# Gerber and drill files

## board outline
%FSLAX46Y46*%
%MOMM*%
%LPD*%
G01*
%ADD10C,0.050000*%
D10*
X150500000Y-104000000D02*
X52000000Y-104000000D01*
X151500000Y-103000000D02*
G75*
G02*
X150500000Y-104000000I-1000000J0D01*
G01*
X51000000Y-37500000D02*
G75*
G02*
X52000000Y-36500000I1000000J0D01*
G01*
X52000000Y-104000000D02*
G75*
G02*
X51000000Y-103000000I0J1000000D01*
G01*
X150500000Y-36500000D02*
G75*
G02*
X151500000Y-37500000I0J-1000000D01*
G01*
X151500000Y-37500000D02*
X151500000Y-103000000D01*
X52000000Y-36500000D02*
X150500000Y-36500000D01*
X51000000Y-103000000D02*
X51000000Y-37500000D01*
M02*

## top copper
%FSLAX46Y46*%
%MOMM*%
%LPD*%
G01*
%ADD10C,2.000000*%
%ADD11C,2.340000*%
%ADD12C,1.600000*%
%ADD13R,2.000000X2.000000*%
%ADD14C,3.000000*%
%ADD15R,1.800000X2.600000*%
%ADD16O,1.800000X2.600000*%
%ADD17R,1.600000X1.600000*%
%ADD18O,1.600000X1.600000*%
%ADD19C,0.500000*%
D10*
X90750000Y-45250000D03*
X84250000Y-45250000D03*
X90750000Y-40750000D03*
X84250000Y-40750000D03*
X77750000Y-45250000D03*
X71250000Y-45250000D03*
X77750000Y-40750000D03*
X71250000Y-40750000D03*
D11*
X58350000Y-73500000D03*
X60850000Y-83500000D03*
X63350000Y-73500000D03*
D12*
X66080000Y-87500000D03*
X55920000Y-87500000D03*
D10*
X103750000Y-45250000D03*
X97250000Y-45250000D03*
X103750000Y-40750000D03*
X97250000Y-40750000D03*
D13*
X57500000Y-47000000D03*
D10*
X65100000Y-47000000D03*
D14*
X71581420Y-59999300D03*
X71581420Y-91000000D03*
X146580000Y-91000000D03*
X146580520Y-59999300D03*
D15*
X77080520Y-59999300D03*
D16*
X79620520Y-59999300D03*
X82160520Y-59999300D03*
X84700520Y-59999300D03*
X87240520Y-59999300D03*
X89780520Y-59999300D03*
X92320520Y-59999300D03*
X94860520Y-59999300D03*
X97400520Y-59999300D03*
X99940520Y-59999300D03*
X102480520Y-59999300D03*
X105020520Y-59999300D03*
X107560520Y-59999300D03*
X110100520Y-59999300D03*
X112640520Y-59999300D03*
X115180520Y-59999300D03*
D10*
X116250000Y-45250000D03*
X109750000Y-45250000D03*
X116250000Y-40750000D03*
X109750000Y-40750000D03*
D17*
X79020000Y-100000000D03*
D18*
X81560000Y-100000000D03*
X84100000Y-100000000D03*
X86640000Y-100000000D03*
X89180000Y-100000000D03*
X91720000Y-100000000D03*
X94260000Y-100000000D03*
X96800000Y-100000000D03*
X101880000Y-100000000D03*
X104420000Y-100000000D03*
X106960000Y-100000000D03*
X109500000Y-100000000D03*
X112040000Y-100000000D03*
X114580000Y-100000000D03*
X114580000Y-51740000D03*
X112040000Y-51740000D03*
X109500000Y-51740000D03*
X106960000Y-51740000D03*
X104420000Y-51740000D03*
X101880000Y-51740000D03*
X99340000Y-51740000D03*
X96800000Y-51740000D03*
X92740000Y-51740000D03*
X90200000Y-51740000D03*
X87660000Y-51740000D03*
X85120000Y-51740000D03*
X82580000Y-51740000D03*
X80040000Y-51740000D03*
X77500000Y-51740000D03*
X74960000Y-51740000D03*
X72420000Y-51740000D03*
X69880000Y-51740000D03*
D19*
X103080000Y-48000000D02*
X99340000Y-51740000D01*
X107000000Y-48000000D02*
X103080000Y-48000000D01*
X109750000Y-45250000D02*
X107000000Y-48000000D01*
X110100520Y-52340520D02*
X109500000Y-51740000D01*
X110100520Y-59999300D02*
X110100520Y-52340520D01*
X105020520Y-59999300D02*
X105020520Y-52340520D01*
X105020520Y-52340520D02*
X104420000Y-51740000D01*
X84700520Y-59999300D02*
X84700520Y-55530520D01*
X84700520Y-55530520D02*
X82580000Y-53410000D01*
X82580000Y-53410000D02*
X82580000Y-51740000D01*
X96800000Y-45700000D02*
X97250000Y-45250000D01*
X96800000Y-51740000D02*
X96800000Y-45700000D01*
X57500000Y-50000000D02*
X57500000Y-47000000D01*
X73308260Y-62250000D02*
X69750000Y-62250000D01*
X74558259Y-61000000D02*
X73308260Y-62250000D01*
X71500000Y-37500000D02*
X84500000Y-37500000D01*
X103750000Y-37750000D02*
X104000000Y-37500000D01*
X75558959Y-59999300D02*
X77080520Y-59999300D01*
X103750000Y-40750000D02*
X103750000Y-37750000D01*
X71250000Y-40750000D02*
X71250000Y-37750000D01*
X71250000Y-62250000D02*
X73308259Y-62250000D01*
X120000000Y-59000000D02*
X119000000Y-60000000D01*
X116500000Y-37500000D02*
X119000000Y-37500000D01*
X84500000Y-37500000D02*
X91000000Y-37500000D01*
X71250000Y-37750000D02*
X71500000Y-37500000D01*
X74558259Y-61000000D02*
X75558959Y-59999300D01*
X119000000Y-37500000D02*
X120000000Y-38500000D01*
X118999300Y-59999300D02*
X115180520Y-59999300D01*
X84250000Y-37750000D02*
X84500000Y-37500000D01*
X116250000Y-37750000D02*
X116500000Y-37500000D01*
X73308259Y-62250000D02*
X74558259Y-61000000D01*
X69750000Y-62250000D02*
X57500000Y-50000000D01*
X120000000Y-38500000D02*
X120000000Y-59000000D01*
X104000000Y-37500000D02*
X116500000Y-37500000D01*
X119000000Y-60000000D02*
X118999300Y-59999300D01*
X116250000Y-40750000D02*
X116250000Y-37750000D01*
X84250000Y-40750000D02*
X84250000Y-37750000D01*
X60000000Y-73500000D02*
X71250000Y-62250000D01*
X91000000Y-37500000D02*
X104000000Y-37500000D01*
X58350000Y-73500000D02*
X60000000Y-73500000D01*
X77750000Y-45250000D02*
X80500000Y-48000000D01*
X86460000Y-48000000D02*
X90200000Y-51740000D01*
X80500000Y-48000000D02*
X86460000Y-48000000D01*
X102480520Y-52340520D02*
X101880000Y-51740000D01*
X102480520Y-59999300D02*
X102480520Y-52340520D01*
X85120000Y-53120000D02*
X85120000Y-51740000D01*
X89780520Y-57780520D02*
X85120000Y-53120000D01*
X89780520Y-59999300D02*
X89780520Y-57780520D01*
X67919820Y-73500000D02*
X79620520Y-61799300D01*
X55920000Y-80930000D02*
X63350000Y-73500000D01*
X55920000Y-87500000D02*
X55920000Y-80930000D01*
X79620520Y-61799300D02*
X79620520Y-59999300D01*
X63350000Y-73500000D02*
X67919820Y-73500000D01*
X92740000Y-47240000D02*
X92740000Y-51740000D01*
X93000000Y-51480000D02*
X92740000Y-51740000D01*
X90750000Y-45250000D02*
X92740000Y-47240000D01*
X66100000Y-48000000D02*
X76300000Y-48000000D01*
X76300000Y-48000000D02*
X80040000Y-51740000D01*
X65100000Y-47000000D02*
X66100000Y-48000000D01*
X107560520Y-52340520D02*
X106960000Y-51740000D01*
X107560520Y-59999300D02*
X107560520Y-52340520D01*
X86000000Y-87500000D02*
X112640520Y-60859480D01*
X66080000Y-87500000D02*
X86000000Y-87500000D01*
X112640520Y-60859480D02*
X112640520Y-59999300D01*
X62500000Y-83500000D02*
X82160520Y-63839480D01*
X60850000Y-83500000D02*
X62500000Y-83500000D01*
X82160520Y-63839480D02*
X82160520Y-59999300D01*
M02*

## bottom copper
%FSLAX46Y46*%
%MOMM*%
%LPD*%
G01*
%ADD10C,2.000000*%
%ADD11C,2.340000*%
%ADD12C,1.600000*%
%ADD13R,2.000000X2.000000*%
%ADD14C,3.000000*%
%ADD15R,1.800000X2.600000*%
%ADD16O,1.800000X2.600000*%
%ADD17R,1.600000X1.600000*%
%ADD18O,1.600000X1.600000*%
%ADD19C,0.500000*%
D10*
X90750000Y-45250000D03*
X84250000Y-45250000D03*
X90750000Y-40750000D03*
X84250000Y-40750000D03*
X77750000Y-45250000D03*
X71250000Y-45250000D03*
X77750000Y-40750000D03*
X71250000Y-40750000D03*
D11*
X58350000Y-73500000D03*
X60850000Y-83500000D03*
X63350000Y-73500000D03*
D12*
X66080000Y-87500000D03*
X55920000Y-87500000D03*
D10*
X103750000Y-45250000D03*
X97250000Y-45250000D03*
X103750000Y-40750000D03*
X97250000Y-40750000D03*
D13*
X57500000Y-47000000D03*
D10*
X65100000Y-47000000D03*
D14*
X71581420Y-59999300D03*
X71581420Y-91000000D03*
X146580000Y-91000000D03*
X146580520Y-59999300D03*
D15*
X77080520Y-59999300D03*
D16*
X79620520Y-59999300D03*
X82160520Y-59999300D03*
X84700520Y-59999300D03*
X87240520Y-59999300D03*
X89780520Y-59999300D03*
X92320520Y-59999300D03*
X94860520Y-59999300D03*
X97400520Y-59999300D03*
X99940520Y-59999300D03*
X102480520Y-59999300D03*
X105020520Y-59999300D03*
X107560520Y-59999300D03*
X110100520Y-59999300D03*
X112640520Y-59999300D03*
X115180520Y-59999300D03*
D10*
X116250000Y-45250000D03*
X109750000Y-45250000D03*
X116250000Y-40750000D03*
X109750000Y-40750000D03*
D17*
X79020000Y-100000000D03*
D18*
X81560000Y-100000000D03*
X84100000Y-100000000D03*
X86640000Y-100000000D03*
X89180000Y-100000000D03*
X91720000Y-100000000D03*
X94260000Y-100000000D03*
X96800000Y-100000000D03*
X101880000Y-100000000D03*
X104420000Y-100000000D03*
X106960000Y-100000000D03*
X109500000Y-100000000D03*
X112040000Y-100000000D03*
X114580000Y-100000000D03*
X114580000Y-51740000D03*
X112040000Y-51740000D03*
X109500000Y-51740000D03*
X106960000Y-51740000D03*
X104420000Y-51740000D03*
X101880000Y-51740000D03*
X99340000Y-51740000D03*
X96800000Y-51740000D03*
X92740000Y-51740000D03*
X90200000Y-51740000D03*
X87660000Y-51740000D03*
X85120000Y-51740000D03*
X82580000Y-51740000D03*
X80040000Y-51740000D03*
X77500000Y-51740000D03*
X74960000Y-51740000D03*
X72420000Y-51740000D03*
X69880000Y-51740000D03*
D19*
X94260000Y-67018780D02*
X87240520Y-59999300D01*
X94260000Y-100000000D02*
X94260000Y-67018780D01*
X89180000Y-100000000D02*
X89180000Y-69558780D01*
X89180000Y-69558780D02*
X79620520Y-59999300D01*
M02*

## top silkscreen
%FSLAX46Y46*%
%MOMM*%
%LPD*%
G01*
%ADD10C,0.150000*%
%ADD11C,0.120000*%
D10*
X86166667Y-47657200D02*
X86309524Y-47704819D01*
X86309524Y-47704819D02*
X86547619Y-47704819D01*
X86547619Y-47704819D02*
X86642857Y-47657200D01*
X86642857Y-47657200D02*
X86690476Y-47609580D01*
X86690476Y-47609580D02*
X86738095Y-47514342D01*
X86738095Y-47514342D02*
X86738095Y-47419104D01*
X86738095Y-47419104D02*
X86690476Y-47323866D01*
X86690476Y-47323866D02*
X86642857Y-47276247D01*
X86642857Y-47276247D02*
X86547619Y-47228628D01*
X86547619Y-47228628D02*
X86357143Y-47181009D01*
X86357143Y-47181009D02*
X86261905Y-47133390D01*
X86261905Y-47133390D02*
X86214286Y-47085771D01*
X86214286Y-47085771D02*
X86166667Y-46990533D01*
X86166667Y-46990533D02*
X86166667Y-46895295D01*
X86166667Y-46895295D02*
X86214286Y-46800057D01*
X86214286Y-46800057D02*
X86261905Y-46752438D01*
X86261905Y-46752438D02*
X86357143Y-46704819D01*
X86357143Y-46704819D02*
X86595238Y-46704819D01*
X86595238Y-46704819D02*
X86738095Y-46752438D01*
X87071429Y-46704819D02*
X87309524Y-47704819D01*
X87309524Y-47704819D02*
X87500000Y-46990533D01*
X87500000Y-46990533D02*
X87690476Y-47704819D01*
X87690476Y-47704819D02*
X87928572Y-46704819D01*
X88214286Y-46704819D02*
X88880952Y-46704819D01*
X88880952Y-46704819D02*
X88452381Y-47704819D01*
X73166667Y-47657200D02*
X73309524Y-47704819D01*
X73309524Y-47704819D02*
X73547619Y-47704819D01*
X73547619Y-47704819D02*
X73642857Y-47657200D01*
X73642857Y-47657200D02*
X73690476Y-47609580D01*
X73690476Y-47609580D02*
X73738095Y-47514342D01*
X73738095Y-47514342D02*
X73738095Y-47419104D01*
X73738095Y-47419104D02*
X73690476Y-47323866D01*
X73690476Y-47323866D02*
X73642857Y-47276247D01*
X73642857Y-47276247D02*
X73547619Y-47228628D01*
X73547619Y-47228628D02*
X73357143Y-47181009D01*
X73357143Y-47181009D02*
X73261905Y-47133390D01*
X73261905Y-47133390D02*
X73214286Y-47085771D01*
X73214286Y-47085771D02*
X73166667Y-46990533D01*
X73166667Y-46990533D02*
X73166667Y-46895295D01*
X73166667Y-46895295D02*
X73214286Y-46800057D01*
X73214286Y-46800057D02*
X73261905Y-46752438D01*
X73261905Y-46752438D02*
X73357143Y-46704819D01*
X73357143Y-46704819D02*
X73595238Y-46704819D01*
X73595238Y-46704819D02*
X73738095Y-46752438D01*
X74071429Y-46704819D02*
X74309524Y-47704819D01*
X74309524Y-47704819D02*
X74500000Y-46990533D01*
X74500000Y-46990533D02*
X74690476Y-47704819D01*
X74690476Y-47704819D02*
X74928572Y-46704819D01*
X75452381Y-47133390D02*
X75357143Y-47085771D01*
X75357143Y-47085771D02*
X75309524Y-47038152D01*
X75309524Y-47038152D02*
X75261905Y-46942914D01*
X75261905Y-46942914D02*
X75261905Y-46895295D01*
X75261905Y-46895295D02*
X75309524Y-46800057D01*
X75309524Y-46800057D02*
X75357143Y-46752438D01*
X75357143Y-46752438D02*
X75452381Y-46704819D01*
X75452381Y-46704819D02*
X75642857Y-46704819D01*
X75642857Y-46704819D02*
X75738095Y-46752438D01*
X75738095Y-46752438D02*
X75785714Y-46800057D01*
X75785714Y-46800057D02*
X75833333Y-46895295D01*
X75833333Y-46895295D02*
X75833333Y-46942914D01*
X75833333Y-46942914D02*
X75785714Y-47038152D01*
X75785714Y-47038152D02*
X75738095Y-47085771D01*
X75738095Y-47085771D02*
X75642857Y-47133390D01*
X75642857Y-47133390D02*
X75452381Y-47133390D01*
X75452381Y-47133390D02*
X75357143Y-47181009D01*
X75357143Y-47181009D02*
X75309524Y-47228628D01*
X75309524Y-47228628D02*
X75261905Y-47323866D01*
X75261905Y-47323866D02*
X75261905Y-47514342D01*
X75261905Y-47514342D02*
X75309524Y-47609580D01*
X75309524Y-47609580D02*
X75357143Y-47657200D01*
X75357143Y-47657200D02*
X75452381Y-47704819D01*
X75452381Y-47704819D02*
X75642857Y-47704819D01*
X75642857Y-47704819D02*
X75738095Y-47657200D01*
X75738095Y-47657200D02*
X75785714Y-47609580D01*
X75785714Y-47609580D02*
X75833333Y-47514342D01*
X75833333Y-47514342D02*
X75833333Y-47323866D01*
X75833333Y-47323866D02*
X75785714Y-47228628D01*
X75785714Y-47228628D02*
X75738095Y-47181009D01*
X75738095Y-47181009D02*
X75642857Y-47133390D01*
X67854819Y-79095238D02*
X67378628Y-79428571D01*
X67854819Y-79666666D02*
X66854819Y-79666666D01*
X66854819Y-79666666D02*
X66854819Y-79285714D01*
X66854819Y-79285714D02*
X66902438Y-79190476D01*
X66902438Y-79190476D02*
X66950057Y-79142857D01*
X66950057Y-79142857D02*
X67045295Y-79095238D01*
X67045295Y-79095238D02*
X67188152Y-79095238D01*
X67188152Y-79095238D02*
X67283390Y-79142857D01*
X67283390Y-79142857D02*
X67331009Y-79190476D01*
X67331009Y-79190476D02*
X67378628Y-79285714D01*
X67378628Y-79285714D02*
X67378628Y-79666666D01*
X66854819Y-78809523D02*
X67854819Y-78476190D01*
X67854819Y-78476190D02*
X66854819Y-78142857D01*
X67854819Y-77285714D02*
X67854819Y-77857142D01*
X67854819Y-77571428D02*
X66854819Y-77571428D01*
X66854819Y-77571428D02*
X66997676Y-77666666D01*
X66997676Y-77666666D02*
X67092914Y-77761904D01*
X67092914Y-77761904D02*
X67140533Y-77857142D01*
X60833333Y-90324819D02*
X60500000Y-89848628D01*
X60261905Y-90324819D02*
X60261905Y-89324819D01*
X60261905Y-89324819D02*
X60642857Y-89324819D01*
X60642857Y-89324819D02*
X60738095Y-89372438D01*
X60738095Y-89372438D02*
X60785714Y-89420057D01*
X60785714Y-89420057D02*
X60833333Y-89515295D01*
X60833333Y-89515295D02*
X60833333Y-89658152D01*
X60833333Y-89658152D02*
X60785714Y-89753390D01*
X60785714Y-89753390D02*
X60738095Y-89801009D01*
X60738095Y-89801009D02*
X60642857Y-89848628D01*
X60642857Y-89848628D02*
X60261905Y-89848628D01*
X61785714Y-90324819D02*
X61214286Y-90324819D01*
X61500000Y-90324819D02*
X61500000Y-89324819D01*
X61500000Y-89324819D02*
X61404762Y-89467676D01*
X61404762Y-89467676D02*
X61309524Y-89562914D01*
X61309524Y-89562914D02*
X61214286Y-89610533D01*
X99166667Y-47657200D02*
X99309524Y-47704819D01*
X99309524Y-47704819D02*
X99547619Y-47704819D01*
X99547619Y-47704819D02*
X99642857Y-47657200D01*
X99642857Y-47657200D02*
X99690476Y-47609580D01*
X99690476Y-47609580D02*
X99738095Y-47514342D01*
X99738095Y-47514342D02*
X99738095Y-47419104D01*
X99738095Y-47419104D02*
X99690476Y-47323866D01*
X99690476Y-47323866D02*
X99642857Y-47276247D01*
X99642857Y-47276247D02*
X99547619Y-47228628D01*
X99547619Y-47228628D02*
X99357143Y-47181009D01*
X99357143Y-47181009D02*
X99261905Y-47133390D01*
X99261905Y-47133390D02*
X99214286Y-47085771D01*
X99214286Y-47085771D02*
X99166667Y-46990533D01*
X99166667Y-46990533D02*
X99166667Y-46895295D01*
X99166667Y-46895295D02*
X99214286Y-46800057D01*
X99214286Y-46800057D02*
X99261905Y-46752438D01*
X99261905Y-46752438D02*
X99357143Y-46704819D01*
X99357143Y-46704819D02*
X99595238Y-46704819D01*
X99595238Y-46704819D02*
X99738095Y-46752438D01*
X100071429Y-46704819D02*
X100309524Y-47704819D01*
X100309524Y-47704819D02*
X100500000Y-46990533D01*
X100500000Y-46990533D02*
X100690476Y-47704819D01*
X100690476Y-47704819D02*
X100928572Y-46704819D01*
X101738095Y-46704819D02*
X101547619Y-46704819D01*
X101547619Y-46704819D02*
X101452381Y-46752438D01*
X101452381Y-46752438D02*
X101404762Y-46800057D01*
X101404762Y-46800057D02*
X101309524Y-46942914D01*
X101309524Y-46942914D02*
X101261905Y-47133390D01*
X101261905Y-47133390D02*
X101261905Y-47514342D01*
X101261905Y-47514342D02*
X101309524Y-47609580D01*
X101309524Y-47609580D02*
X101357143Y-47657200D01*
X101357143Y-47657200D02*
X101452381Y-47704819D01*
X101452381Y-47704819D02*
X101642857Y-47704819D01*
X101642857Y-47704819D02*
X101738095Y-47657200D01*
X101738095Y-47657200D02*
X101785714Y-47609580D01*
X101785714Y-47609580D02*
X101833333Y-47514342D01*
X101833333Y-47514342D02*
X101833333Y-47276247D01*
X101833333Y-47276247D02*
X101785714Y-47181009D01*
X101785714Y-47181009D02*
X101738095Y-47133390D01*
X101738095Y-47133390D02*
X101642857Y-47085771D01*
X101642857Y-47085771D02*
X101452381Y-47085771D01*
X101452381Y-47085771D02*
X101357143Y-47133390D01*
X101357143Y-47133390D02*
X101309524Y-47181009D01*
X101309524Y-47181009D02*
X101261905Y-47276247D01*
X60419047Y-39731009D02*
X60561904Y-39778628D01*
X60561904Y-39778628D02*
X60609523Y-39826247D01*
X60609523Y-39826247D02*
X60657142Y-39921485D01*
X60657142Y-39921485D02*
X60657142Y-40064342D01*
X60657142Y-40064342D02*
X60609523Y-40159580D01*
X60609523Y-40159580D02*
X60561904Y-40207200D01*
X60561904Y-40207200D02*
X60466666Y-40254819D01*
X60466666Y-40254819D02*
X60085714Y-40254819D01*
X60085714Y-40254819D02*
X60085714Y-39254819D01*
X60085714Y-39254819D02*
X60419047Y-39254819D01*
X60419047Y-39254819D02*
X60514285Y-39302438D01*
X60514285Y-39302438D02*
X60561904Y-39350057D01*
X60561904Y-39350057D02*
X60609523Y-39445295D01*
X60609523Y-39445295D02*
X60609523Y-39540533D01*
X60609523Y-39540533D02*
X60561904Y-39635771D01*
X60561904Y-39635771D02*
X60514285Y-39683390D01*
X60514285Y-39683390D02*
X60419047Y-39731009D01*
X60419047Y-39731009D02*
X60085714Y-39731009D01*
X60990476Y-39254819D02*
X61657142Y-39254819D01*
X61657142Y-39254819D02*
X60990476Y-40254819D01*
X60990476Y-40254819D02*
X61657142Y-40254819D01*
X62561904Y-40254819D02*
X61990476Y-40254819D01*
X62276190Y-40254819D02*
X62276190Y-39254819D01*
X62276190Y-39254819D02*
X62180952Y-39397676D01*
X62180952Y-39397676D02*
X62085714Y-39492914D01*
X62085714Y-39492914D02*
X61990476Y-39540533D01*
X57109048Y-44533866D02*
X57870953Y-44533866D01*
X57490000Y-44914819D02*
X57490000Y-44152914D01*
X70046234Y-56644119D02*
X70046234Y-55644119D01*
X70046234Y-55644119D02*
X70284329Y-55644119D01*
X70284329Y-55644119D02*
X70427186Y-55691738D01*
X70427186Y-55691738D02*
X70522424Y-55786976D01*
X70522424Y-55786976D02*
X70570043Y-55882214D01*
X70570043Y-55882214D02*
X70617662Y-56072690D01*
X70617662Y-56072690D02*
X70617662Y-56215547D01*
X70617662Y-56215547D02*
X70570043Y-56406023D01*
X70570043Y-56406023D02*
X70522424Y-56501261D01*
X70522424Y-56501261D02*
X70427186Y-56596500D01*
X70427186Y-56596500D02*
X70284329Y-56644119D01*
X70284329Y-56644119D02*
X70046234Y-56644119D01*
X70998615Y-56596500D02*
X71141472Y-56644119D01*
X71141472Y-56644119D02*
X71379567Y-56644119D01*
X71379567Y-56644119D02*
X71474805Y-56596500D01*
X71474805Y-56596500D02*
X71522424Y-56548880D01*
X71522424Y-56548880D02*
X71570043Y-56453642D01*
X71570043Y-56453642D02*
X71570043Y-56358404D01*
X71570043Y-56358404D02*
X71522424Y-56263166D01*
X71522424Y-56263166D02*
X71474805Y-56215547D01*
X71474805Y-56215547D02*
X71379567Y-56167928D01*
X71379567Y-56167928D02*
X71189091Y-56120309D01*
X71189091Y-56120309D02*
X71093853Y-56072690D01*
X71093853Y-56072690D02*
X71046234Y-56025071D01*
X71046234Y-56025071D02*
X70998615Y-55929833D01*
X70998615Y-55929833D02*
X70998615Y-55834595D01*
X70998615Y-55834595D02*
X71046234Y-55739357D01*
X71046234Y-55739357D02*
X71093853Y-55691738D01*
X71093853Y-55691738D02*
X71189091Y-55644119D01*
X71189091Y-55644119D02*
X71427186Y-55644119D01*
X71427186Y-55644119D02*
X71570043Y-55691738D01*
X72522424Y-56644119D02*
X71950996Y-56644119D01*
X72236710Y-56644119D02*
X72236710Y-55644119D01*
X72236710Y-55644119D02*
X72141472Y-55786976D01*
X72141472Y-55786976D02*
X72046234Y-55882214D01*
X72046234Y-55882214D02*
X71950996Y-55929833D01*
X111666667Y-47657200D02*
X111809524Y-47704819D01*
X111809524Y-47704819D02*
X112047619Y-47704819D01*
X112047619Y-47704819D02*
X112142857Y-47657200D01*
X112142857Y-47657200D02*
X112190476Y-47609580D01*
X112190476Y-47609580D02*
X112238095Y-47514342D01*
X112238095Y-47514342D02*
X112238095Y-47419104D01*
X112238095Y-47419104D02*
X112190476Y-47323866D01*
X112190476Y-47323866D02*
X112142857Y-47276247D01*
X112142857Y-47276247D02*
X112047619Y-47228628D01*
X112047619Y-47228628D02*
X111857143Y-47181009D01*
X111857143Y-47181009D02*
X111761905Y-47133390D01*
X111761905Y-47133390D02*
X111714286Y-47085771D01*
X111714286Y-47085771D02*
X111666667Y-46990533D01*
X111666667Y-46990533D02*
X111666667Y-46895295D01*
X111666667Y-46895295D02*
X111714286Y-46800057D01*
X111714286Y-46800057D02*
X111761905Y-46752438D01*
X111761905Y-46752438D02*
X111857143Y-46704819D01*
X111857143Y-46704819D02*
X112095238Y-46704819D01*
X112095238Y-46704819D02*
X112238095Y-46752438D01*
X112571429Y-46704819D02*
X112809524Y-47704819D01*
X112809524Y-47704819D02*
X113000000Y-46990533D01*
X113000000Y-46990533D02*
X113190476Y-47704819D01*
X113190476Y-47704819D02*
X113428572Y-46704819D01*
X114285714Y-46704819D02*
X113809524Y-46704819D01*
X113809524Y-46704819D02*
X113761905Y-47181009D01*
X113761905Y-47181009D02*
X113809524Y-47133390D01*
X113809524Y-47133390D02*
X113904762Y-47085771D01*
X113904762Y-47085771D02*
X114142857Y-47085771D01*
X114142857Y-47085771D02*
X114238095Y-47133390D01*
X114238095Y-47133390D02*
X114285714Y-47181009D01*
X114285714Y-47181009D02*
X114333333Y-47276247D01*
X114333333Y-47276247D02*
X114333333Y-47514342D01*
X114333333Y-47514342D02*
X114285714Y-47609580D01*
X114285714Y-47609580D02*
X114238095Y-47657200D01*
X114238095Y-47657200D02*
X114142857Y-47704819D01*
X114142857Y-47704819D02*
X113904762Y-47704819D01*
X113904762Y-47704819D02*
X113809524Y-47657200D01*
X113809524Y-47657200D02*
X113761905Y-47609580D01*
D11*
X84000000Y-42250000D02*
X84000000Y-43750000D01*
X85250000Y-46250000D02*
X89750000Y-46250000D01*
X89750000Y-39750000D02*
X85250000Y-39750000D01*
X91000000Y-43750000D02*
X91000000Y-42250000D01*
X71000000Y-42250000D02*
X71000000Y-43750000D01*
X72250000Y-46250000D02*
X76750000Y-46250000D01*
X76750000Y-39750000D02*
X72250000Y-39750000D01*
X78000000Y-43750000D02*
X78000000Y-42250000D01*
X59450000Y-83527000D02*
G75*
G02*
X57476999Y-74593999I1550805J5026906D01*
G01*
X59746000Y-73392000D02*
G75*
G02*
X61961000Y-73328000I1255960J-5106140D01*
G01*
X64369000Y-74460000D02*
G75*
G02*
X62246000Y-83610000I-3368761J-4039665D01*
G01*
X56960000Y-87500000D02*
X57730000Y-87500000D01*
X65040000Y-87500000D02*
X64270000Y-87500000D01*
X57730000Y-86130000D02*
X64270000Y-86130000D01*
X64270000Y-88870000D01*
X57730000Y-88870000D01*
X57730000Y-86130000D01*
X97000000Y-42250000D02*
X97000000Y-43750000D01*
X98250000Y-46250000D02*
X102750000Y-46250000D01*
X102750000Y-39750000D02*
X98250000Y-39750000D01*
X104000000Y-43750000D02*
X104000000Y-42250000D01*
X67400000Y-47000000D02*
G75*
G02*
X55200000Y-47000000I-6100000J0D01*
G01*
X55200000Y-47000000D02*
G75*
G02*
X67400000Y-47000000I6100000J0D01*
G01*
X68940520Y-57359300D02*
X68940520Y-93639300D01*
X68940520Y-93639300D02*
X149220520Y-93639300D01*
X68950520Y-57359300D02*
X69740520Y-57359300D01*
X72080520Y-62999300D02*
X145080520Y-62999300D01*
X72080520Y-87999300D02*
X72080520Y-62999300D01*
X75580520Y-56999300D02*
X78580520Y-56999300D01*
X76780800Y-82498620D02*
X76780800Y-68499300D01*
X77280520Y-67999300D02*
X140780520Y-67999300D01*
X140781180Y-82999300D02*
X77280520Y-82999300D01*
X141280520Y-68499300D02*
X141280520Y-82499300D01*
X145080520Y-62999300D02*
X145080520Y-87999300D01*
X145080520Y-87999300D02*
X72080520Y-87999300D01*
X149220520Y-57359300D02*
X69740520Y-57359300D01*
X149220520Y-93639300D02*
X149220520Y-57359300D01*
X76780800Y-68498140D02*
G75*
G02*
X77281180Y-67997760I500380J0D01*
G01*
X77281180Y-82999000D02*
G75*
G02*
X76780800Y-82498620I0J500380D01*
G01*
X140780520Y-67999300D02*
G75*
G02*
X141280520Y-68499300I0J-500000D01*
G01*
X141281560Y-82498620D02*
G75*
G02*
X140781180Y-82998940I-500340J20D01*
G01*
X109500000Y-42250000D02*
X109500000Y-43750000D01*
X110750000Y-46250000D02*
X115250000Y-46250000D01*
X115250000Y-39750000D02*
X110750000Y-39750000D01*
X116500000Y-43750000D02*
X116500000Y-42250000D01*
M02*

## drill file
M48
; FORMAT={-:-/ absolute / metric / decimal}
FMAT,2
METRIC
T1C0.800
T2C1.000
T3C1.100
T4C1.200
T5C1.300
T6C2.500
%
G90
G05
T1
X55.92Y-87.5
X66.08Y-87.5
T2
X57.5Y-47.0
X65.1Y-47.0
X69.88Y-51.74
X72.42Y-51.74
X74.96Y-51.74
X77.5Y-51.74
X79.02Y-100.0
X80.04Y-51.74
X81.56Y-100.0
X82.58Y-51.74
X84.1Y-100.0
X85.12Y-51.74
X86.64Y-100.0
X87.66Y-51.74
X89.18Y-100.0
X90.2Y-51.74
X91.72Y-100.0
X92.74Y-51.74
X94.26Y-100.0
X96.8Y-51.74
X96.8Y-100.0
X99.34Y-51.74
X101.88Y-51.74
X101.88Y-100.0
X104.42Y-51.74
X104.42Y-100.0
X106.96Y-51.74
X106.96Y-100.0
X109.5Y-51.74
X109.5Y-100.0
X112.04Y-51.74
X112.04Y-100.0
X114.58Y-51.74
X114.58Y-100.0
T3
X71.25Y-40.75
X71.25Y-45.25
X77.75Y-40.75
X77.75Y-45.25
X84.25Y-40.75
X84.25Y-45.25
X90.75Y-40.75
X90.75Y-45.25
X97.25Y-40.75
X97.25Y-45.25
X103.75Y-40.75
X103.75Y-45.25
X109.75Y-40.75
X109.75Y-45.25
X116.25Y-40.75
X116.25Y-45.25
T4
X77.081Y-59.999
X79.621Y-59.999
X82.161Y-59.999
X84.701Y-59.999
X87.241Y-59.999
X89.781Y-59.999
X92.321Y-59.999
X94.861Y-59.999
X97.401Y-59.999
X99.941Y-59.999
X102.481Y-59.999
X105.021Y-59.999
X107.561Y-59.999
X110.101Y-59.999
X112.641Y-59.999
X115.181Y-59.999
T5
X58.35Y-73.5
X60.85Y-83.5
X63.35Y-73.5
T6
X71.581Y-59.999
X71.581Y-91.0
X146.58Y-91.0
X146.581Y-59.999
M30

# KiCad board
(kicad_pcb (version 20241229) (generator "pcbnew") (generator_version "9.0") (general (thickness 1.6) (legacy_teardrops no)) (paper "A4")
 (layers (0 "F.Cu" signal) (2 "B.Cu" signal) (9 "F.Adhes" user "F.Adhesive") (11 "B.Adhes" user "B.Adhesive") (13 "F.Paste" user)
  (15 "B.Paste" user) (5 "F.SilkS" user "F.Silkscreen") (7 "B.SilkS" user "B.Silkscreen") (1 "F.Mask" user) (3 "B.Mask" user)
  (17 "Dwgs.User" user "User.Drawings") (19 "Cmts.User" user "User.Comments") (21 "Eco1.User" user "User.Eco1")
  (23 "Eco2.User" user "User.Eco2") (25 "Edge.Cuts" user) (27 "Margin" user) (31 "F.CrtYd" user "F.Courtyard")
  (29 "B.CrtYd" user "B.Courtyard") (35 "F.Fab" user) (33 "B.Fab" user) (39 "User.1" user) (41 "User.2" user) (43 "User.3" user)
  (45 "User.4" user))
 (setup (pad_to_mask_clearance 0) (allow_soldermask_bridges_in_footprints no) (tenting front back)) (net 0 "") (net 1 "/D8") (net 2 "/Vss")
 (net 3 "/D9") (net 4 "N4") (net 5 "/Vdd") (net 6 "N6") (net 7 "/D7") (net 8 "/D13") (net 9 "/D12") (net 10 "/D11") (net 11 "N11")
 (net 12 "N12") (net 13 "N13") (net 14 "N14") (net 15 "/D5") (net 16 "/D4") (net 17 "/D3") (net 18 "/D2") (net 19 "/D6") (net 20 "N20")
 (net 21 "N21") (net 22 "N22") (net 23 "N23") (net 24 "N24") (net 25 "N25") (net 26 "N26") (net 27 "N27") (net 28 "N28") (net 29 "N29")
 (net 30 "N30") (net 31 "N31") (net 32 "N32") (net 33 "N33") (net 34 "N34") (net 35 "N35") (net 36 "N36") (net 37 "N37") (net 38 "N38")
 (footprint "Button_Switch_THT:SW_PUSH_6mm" (layer "F.Cu") (at 90.75 45.25 180)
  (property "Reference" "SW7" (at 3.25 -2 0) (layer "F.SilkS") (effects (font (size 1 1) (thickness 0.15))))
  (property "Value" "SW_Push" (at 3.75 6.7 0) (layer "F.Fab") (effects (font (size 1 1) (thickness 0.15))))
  (fp_line (start 6.75 3) (end 6.75 1.5) (stroke (width 0.12) (type solid)) (layer "F.SilkS"))
  (fp_line (start 5.5 -1) (end 1 -1) (stroke (width 0.12) (type solid)) (layer "F.SilkS"))
  (fp_line (start 1 5.5) (end 5.5 5.5) (stroke (width 0.12) (type solid)) (layer "F.SilkS"))
  (fp_line (start -0.25 1.5) (end -0.25 3) (stroke (width 0.12) (type solid)) (layer "F.SilkS"))
  (pad "1" thru_hole circle (at 0 0 270) (size 2 2) (drill 1.1) (layers "*.Cu" "*.Mask") (remove_unused_layers no) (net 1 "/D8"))
  (pad "1" thru_hole circle (at 6.5 0 270) (size 2 2) (drill 1.1) (layers "*.Cu" "*.Mask") (remove_unused_layers no) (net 1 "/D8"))
  (pad "2" thru_hole circle (at 0 4.5 270) (size 2 2) (drill 1.1) (layers "*.Cu" "*.Mask") (remove_unused_layers no) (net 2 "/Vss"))
  (pad "2" thru_hole circle (at 6.5 4.5 270) (size 2 2) (drill 1.1) (layers "*.Cu" "*.Mask") (remove_unused_layers no) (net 2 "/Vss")))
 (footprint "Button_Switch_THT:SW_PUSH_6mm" (layer "F.Cu") (at 77.75 45.25 180)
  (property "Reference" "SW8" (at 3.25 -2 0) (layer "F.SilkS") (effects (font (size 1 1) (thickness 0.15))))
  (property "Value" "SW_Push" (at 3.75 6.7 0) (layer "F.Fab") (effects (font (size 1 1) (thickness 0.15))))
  (fp_line (start 6.75 3) (end 6.75 1.5) (stroke (width 0.12) (type solid)) (layer "F.SilkS"))
  (fp_line (start 5.5 -1) (end 1 -1) (stroke (width 0.12) (type solid)) (layer "F.SilkS"))
  (fp_line (start 1 5.5) (end 5.5 5.5) (stroke (width 0.12) (type solid)) (layer "F.SilkS"))
  (fp_line (start -0.25 1.5) (end -0.25 3) (stroke (width 0.12) (type solid)) (layer "F.SilkS"))
  (pad "1" thru_hole circle (at 0 0 270) (size 2 2) (drill 1.1) (layers "*.Cu" "*.Mask") (remove_unused_layers no) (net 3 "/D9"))
  (pad "1" thru_hole circle (at 6.5 0 270) (size 2 2) (drill 1.1) (layers "*.Cu" "*.Mask") (remove_unused_layers no) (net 3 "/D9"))
  (pad "2" thru_hole circle (at 0 4.5 270) (size 2 2) (drill 1.1) (layers "*.Cu" "*.Mask") (remove_unused_layers no) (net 2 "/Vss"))
  (pad "2" thru_hole circle (at 6.5 4.5 270) (size 2 2) (drill 1.1) (layers "*.Cu" "*.Mask") (remove_unused_layers no) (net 2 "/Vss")))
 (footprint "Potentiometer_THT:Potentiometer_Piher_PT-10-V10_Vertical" (layer "F.Cu") (at 58.35 73.5 -90)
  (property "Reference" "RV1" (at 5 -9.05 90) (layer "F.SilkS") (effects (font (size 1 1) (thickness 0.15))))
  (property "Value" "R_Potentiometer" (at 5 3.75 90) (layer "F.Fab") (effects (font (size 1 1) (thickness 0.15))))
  (fp_arc (start 10.027 -1.1) (mid 6.134659 2.486075) (end 1.094 0.873) (stroke (width 0.12) (type solid)) (layer "F.SilkS"))
  (fp_arc (start -0.108 -1.396) (mid -0.258003 -2.50009) (end -0.172 -3.611) (stroke (width 0.12) (type solid)) (layer "F.SilkS"))
  (fp_arc (start 0.96 -6.019) (mid 6.188516 -7.774112) (end 10.11 -3.896) (stroke (width 0.12) (type solid)) (layer "F.SilkS"))
  (pad "1" thru_hole circle (at 0 0 270) (size 2.34 2.34) (drill 1.3) (layers "*.Cu" "*.Mask") (remove_unused_layers no) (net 2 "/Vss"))
  (pad "2" thru_hole circle (at 10 -2.5 270) (size 2.34 2.34) (drill 1.3) (layers "*.Cu" "*.Mask") (remove_unused_layers no) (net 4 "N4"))
  (pad "3" thru_hole circle (at 0 -5 270) (size 2.34 2.34) (drill 1.3) (layers "*.Cu" "*.Mask") (remove_unused_layers no) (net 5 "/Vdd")))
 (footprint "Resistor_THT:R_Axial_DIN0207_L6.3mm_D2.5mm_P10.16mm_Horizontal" (layer "F.Cu") (at 66.08 87.5 180)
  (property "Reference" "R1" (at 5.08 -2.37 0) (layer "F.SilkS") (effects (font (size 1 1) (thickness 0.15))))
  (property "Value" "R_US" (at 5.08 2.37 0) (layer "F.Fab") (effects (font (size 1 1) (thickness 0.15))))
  (fp_line (start 9.12 0) (end 8.35 0) (stroke (width 0.12) (type solid)) (layer "F.SilkS"))
  (fp_line (start 1.04 0) (end 1.81 0) (stroke (width 0.12) (type solid)) (layer "F.SilkS"))
  (fp_rect (start 1.81 -1.37) (end 8.35 1.37) (stroke (width 0.12) (type solid)) (fill no) (layer "F.SilkS"))
  (pad "1" thru_hole circle (at 0 0 180) (size 1.6 1.6) (drill 0.8) (layers "*.Cu" "*.Mask") (remove_unused_layers no) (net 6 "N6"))
  (pad "2" thru_hole circle (at 10.16 0 180) (size 1.6 1.6) (drill 0.8) (layers "*.Cu" "*.Mask") (remove_unused_layers no) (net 5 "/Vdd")))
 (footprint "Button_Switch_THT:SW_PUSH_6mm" (layer "F.Cu") (at 103.75 45.25 180)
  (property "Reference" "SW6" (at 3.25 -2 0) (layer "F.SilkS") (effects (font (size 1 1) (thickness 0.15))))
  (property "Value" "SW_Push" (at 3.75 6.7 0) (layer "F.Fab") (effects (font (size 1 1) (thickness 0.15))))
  (fp_line (start 6.75 3) (end 6.75 1.5) (stroke (width 0.12) (type solid)) (layer "F.SilkS"))
  (fp_line (start 5.5 -1) (end 1 -1) (stroke (width 0.12) (type solid)) (layer "F.SilkS"))
  (fp_line (start 1 5.5) (end 5.5 5.5) (stroke (width 0.12) (type solid)) (layer "F.SilkS"))
  (fp_line (start -0.25 1.5) (end -0.25 3) (stroke (width 0.12) (type solid)) (layer "F.SilkS"))
  (pad "1" thru_hole circle (at 0 0 270) (size 2 2) (drill 1.1) (layers "*.Cu" "*.Mask") (remove_unused_layers no) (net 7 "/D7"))
  (pad "1" thru_hole circle (at 6.5 0 270) (size 2 2) (drill 1.1) (layers "*.Cu" "*.Mask") (remove_unused_layers no) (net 7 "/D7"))
  (pad "2" thru_hole circle (at 0 4.5 270) (size 2 2) (drill 1.1) (layers "*.Cu" "*.Mask") (remove_unused_layers no) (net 2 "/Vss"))
  (pad "2" thru_hole circle (at 6.5 4.5 270) (size 2 2) (drill 1.1) (layers "*.Cu" "*.Mask") (remove_unused_layers no) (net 2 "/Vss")))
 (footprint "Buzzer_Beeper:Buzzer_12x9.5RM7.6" (layer "F.Cu") (at 57.5 47)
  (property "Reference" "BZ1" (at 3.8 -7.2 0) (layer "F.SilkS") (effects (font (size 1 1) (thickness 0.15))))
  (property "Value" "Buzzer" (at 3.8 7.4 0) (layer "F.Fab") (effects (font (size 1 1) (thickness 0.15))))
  (fp_circle (center 3.8 0) (end 9.9 0) (stroke (width 0.12) (type solid)) (fill no) (layer "F.SilkS"))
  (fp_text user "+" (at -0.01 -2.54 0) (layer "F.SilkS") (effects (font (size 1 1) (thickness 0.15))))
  (pad "1" thru_hole rect (at 0 0) (size 2 2) (drill 1) (layers "*.Cu" "*.Mask") (remove_unused_layers no) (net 2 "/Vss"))
  (pad "2" thru_hole circle (at 7.6 0) (size 2 2) (drill 1) (layers "*.Cu" "*.Mask") (remove_unused_layers no) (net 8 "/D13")))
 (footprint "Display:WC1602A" (layer "F.Cu") (at 77.08052 59.9993)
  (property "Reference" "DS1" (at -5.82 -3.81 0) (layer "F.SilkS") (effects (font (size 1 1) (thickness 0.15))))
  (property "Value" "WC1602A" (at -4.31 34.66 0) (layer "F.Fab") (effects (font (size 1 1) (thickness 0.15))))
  (fp_line (start -8.14 -2.64) (end -8.14 33.64) (stroke (width 0.12) (type solid)) (layer "F.SilkS"))
  (fp_line (start -8.14 33.64) (end 72.14 33.64) (stroke (width 0.12) (type solid)) (layer "F.SilkS"))
  (fp_line (start -8.13 -2.64) (end -7.34 -2.64) (stroke (width 0.12) (type solid)) (layer "F.SilkS"))
  (fp_line (start -5 3) (end 68 3) (stroke (width 0.12) (type solid)) (layer "F.SilkS"))
  (fp_line (start -5 28) (end -5 3) (stroke (width 0.12) (type solid)) (layer "F.SilkS"))
  (fp_line (start -1.5 -3) (end 1.5 -3) (stroke (width 0.12) (type solid)) (layer "F.SilkS"))
  (fp_line (start -0.29972 22.49932) (end -0.29972 8.5) (stroke (width 0.12) (type solid)) (layer "F.SilkS"))
  (fp_line (start 0.2 8) (end 63.7 8) (stroke (width 0.12) (type solid)) (layer "F.SilkS"))
  (fp_line (start 63.70066 23) (end 0.2 23) (stroke (width 0.12) (type solid)) (layer "F.SilkS"))
  (fp_line (start 64.2 8.5) (end 64.2 22.5) (stroke (width 0.12) (type solid)) (layer "F.SilkS"))
  (fp_line (start 68 3) (end 68 28) (stroke (width 0.12) (type solid)) (layer "F.SilkS"))
  (fp_line (start 68 28) (end -5 28) (stroke (width 0.12) (type solid)) (layer "F.SilkS"))
  (fp_line (start 72.14 -2.64) (end -7.34 -2.64) (stroke (width 0.12) (type solid)) (layer "F.SilkS"))
  (fp_line (start 72.14 33.64) (end 72.14 -2.64) (stroke (width 0.12) (type solid)) (layer "F.SilkS"))
  (fp_arc (start -0.29972 8.49884) (mid -0.153162 8.145018) (end 0.20066 7.99846) (stroke (width 0.12) (type solid)) (layer "F.SilkS"))
  (fp_arc (start 0.20066 22.9997) (mid -0.153162 22.853142) (end -0.29972 22.49932) (stroke (width 0.12) (type solid)) (layer "F.SilkS"))
  (fp_arc (start 63.7 8) (mid 64.053553 8.146447) (end 64.2 8.5) (stroke (width 0.12) (type solid)) (layer "F.SilkS"))
  (fp_arc (start 64.20104 22.49932) (mid 64.054482 22.853142) (end 63.70066 22.9997) (stroke (width 0.12) (type solid)) (layer "F.SilkS"))
  (pad "" thru_hole circle (at -5.4991 0) (size 3 3) (drill 2.5) (layers "*.Cu" "*.Mask") (remove_unused_layers no))
  (pad "" thru_hole circle (at -5.4991 31.0007) (size 3 3) (drill 2.5) (layers "*.Cu" "*.Mask") (remove_unused_layers no))
  (pad "" thru_hole circle (at 69.49948 31.0007) (size 3 3) (drill 2.5) (layers "*.Cu" "*.Mask") (remove_unused_layers no))
  (pad "" thru_hole circle (at 69.5 0) (size 3 3) (drill 2.5) (layers "*.Cu" "*.Mask") (remove_unused_layers no))
  (pad "1" thru_hole rect (at 0 0) (size 1.8 2.6) (drill 1.2) (layers "*.Cu" "*.Mask") (remove_unused_layers no) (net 2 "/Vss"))
  (pad "2" thru_hole oval (at 2.54 0) (size 1.8 2.6) (drill 1.2) (layers "*.Cu" "*.Mask") (remove_unused_layers no) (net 5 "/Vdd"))
  (pad "3" thru_hole oval (at 5.08 0) (size 1.8 2.6) (drill 1.2) (layers "*.Cu" "*.Mask") (remove_unused_layers no) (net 4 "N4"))
  (pad "4" thru_hole oval (at 7.62 0) (size 1.8 2.6) (drill 1.2) (layers "*.Cu" "*.Mask") (remove_unused_layers no) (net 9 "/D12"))
  (pad "5" thru_hole oval (at 10.16 0) (size 1.8 2.6) (drill 1.2) (layers "*.Cu" "*.Mask") (remove_unused_layers no) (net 2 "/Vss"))
  (pad "6" thru_hole oval (at 12.7 0) (size 1.8 2.6) (drill 1.2) (layers "*.Cu" "*.Mask") (remove_unused_layers no) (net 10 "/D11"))
  (pad "7" thru_hole oval (at 15.24 0) (size 1.8 2.6) (drill 1.2) (layers "*.Cu" "*.Mask") (remove_unused_layers no) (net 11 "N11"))
  (pad "8" thru_hole oval (at 17.78 0) (size 1.8 2.6) (drill 1.2) (layers "*.Cu" "*.Mask") (remove_unused_layers no) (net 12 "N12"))
  (pad "9" thru_hole oval (at 20.32 0) (size 1.8 2.6) (drill 1.2) (layers "*.Cu" "*.Mask") (remove_unused_layers no) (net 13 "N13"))
  (pad "10" thru_hole oval (at 22.86 0) (size 1.8 2.6) (drill 1.2) (layers "*.Cu" "*.Mask") (remove_unused_layers no) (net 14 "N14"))
  (pad "11" thru_hole oval (at 25.4 0) (size 1.8 2.6) (drill 1.2) (layers "*.Cu" "*.Mask") (remove_unused_layers no) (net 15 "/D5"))
  (pad "12" thru_hole oval (at 27.94 0) (size 1.8 2.6) (drill 1.2) (layers "*.Cu" "*.Mask") (remove_unused_layers no) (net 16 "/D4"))
  (pad "13" thru_hole oval (at 30.48 0) (size 1.8 2.6) (drill 1.2) (layers "*.Cu" "*.Mask") (remove_unused_layers no) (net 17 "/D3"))
  (pad "14" thru_hole oval (at 33.02 0) (size 1.8 2.6) (drill 1.2) (layers "*.Cu" "*.Mask") (remove_unused_layers no) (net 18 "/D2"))
  (pad "15" thru_hole oval (at 35.56 0) (size 1.8 2.6) (drill 1.2) (layers "*.Cu" "*.Mask") (remove_unused_layers no) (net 6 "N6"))
  (pad "16" thru_hole oval (at 38.1 0) (size 1.8 2.6) (drill 1.2) (layers "*.Cu" "*.Mask") (remove_unused_layers no) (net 2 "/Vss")))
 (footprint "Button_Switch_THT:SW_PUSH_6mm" (layer "F.Cu") (at 116.25 45.25 180)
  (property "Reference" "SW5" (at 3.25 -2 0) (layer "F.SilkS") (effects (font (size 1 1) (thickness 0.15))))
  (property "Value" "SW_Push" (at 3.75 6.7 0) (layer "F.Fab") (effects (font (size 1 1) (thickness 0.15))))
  (fp_line (start 6.75 3) (end 6.75 1.5) (stroke (width 0.12) (type solid)) (layer "F.SilkS"))
  (fp_line (start 5.5 -1) (end 1 -1) (stroke (width 0.12) (type solid)) (layer "F.SilkS"))
  (fp_line (start 1 5.5) (end 5.5 5.5) (stroke (width 0.12) (type solid)) (layer "F.SilkS"))
  (fp_line (start -0.25 1.5) (end -0.25 3) (stroke (width 0.12) (type solid)) (layer "F.SilkS"))
  (pad "1" thru_hole circle (at 0 0 270) (size 2 2) (drill 1.1) (layers "*.Cu" "*.Mask") (remove_unused_layers no) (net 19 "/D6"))
  (pad "1" thru_hole circle (at 6.5 0 270) (size 2 2) (drill 1.1) (layers "*.Cu" "*.Mask") (remove_unused_layers no) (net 19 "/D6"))
  (pad "2" thru_hole circle (at 0 4.5 270) (size 2 2) (drill 1.1) (layers "*.Cu" "*.Mask") (remove_unused_layers no) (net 2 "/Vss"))
  (pad "2" thru_hole circle (at 6.5 4.5 270) (size 2 2) (drill 1.1) (layers "*.Cu" "*.Mask") (remove_unused_layers no) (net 2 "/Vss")))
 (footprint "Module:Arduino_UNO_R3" (layer "B.Cu") (at 79.02 100)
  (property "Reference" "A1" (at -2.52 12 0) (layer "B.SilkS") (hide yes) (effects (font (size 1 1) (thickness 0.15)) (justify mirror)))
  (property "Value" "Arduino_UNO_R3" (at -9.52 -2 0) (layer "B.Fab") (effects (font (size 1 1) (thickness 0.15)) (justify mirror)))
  (pad "1" thru_hole rect (at 0 0 270) (size 1.6 1.6) (drill 1) (layers "*.Cu" "*.Mask") (remove_unused_layers no) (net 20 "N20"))
  (pad "2" thru_hole oval (at 2.54 0 270) (size 1.6 1.6) (drill 1) (layers "*.Cu" "*.Mask") (remove_unused_layers no) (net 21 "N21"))
  (pad "3" thru_hole oval (at 5.08 0 270) (size 1.6 1.6) (drill 1) (layers "*.Cu" "*.Mask") (remove_unused_layers no) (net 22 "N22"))
  (pad "4" thru_hole oval (at 7.62 0 270) (size 1.6 1.6) (drill 1) (layers "*.Cu" "*.Mask") (remove_unused_layers no) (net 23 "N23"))
  (pad "5" thru_hole oval (at 10.16 0 270) (size 1.6 1.6) (drill 1) (layers "*.Cu" "*.Mask") (remove_unused_layers no) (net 5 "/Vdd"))
  (pad "6" thru_hole oval (at 12.7 0 270) (size 1.6 1.6) (drill 1) (layers "*.Cu" "*.Mask") (remove_unused_layers no) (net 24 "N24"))
  (pad "7" thru_hole oval (at 15.24 0 270) (size 1.6 1.6) (drill 1) (layers "*.Cu" "*.Mask") (remove_unused_layers no) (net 2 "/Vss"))
  (pad "8" thru_hole oval (at 17.78 0 270) (size 1.6 1.6) (drill 1) (layers "*.Cu" "*.Mask") (remove_unused_layers no) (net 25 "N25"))
  (pad "9" thru_hole oval (at 22.86 0 270) (size 1.6 1.6) (drill 1) (layers "*.Cu" "*.Mask") (remove_unused_layers no) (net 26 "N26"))
  (pad "10" thru_hole oval (at 25.4 0 270) (size 1.6 1.6) (drill 1) (layers "*.Cu" "*.Mask") (remove_unused_layers no) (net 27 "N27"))
  (pad "11" thru_hole oval (at 27.94 0 270) (size 1.6 1.6) (drill 1) (layers "*.Cu" "*.Mask") (remove_unused_layers no) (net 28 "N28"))
  (pad "12" thru_hole oval (at 30.48 0 270) (size 1.6 1.6) (drill 1) (layers "*.Cu" "*.Mask") (remove_unused_layers no) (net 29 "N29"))
  (pad "13" thru_hole oval (at 33.02 0 270) (size 1.6 1.6) (drill 1) (layers "*.Cu" "*.Mask") (remove_unused_layers no) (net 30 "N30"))
  (pad "14" thru_hole oval (at 35.56 0 270) (size 1.6 1.6) (drill 1) (layers "*.Cu" "*.Mask") (remove_unused_layers no) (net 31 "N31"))
  (pad "15" thru_hole oval (at 35.56 -48.26 270) (size 1.6 1.6) (drill 1) (layers "*.Cu" "*.Mask") (remove_unused_layers no) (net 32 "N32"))
  (pad "16" thru_hole oval (at 33.02 -48.26 270) (size 1.6 1.6) (drill 1) (layers "*.Cu" "*.Mask") (remove_unused_layers no) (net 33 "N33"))
  (pad "17" thru_hole oval (at 30.48 -48.26 270) (size 1.6 1.6) (drill 1) (layers "*.Cu" "*.Mask") (remove_unused_layers no) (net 18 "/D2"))
  (pad "18" thru_hole oval (at 27.94 -48.26 270) (size 1.6 1.6) (drill 1) (layers "*.Cu" "*.Mask") (remove_unused_layers no) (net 17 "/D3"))
  (pad "19" thru_hole oval (at 25.4 -48.26 270) (size 1.6 1.6) (drill 1) (layers "*.Cu" "*.Mask") (remove_unused_layers no) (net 16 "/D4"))
  (pad "20" thru_hole oval (at 22.86 -48.26 270) (size 1.6 1.6) (drill 1) (layers "*.Cu" "*.Mask") (remove_unused_layers no) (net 15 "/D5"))
  (pad "21" thru_hole oval (at 20.32 -48.26 270) (size 1.6 1.6) (drill 1) (layers "*.Cu" "*.Mask") (remove_unused_layers no) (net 19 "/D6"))
  (pad "22" thru_hole oval (at 17.78 -48.26 270) (size 1.6 1.6) (drill 1) (layers "*.Cu" "*.Mask") (remove_unused_layers no) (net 7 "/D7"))
  (pad "23" thru_hole oval (at 13.72 -48.26 270) (size 1.6 1.6) (drill 1) (layers "*.Cu" "*.Mask") (remove_unused_layers no) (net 1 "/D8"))
  (pad "24" thru_hole oval (at 11.18 -48.26 270) (size 1.6 1.6) (drill 1) (layers "*.Cu" "*.Mask") (remove_unused_layers no) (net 3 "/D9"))
  (pad "25" thru_hole oval (at 8.64 -48.26 270) (size 1.6 1.6) (drill 1) (layers "*.Cu" "*.Mask") (remove_unused_layers no) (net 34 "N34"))
  (pad "26" thru_hole oval (at 6.1 -48.26 270) (size 1.6 1.6) (drill 1) (layers "*.Cu" "*.Mask") (remove_unused_layers no) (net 10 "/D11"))
  (pad "27" thru_hole oval (at 3.56 -48.26 270) (size 1.6 1.6) (drill 1) (layers "*.Cu" "*.Mask") (remove_unused_layers no) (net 9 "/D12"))
  (pad "28" thru_hole oval (at 1.02 -48.26 270) (size 1.6 1.6) (drill 1) (layers "*.Cu" "*.Mask") (remove_unused_layers no) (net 8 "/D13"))
  (pad "29" thru_hole oval (at -1.52 -48.26 270) (size 1.6 1.6) (drill 1) (layers "*.Cu" "*.Mask") (remove_unused_layers no) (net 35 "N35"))
  (pad "30" thru_hole oval (at -4.06 -48.26 270) (size 1.6 1.6) (drill 1) (layers "*.Cu" "*.Mask") (remove_unused_layers no) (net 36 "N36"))
  (pad "31" thru_hole oval (at -6.6 -48.26 270) (size 1.6 1.6) (drill 1) (layers "*.Cu" "*.Mask") (remove_unused_layers no) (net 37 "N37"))
  (pad "32" thru_hole oval (at -9.14 -48.26 270) (size 1.6 1.6) (drill 1) (layers "*.Cu" "*.Mask") (remove_unused_layers no) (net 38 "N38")))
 (gr_line (start 150.5 104) (end 52 104) (stroke (width 0.05) (type default)) (layer "Edge.Cuts"))
 (gr_arc (start 151.5 103) (mid 151.207107 103.707107) (end 150.5 104) (stroke (width 0.05) (type default)) (layer "Edge.Cuts"))
 (gr_arc (start 51 37.5) (mid 51.292893 36.792893) (end 52 36.5) (stroke (width 0.05) (type default)) (layer "Edge.Cuts"))
 (gr_arc (start 52 104) (mid 51.292893 103.707107) (end 51 103) (stroke (width 0.05) (type default)) (layer "Edge.Cuts"))
 (gr_arc (start 150.5 36.5) (mid 151.207107 36.792893) (end 151.5 37.5) (stroke (width 0.05) (type default)) (layer "Edge.Cuts"))
 (gr_line (start 151.5 37.5) (end 151.5 103) (stroke (width 0.05) (type default)) (layer "Edge.Cuts"))
 (gr_line (start 52 36.5) (end 150.5 36.5) (stroke (width 0.05) (type default)) (layer "Edge.Cuts"))
 (gr_line (start 51 103) (end 51 37.5) (stroke (width 0.05) (type default)) (layer "Edge.Cuts"))
 (segment (start 103.08 48) (end 99.34 51.74) (width 0.5) (layer "F.Cu") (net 19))
 (segment (start 107 48) (end 103.08 48) (width 0.5) (layer "F.Cu") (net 19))
 (segment (start 109.75 45.25) (end 107 48) (width 0.5) (layer "F.Cu") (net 19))
 (segment (start 110.10052 52.34052) (end 109.5 51.74) (width 0.5) (layer "F.Cu") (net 18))
 (segment (start 110.10052 59.9993) (end 110.10052 52.34052) (width 0.5) (layer "F.Cu") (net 18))
 (segment (start 105.02052 59.9993) (end 105.02052 52.34052) (width 0.5) (layer "F.Cu") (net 16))
 (segment (start 105.02052 52.34052) (end 104.42 51.74) (width 0.5) (layer "F.Cu") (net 16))
 (segment (start 84.70052 59.9993) (end 84.70052 55.53052) (width 0.5) (layer "F.Cu") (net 9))
 (segment (start 84.70052 55.53052) (end 82.58 53.41) (width 0.5) (layer "F.Cu") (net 9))
 (segment (start 82.58 53.41) (end 82.58 51.74) (width 0.5) (layer "F.Cu") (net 9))
 (segment (start 96.8 45.7) (end 97.25 45.25) (width 0.5) (layer "F.Cu") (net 7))
 (segment (start 96.8 51.74) (end 96.8 45.7) (width 0.5) (layer "F.Cu") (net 7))
 (segment (start 57.5 50) (end 57.5 47) (width 0.5) (layer "F.Cu") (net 2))
 (segment (start 73.30826 62.25) (end 69.75 62.25) (width 0.5) (layer "F.Cu") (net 2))
 (segment (start 74.558259 61) (end 73.30826 62.25) (width 0.5) (layer "F.Cu") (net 2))
 (segment (start 71.5 37.5) (end 84.5 37.5) (width 0.5) (layer "F.Cu") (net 2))
 (segment (start 103.75 37.75) (end 104 37.5) (width 0.5) (layer "F.Cu") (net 2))
 (segment (start 75.558959 59.9993) (end 77.08052 59.9993) (width 0.5) (layer "F.Cu") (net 2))
 (segment (start 103.75 40.75) (end 103.75 37.75) (width 0.5) (layer "F.Cu") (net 2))
 (segment (start 71.25 40.75) (end 71.25 37.75) (width 0.5) (layer "F.Cu") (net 2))
 (segment (start 71.25 62.25) (end 73.308259 62.25) (width 0.5) (layer "F.Cu") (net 2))
 (segment (start 120 59) (end 119 60) (width 0.5) (layer "F.Cu") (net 2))
 (segment (start 116.5 37.5) (end 119 37.5) (width 0.5) (layer "F.Cu") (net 2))
 (segment (start 84.5 37.5) (end 91 37.5) (width 0.5) (layer "F.Cu") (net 2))
 (segment (start 71.25 37.75) (end 71.5 37.5) (width 0.5) (layer "F.Cu") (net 2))
 (segment (start 74.558259 61) (end 75.558959 59.9993) (width 0.5) (layer "F.Cu") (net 2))
 (segment (start 119 37.5) (end 120 38.5) (width 0.5) (layer "F.Cu") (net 2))
 (segment (start 118.9993 59.9993) (end 115.18052 59.9993) (width 0.5) (layer "F.Cu") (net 2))
 (segment (start 84.25 37.75) (end 84.5 37.5) (width 0.5) (layer "F.Cu") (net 2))
 (segment (start 116.25 37.75) (end 116.5 37.5) (width 0.5) (layer "F.Cu") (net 2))
 (segment (start 73.308259 62.25) (end 74.558259 61) (width 0.5) (layer "F.Cu") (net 2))
 (segment (start 69.75 62.25) (end 57.5 50) (width 0.5) (layer "F.Cu") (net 2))
 (segment (start 120 38.5) (end 120 59) (width 0.5) (layer "F.Cu") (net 2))
 (segment (start 104 37.5) (end 116.5 37.5) (width 0.5) (layer "F.Cu") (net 2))
 (segment (start 119 60) (end 118.9993 59.9993) (width 0.5) (layer "F.Cu") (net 2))
 (segment (start 116.25 40.75) (end 116.25 37.75) (width 0.5) (layer "F.Cu") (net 2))
 (segment (start 84.25 40.75) (end 84.25 37.75) (width 0.5) (layer "F.Cu") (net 2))
 (segment (start 60 73.5) (end 71.25 62.25) (width 0.5) (layer "F.Cu") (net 2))
 (segment (start 91 37.5) (end 104 37.5) (width 0.5) (layer "F.Cu") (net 2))
 (segment (start 58.35 73.5) (end 60 73.5) (width 0.5) (layer "F.Cu") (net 2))
 (segment (start 94.26 67.01878) (end 87.24052 59.9993) (width 0.5) (layer "B.Cu") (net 2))
 (segment (start 94.26 100) (end 94.26 67.01878) (width 0.5) (layer "B.Cu") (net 2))
 (segment (start 77.75 45.25) (end 80.5 48) (width 0.5) (layer "F.Cu") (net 3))
 (segment (start 86.46 48) (end 90.2 51.74) (width 0.5) (layer "F.Cu") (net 3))
 (segment (start 80.5 48) (end 86.46 48) (width 0.5) (layer "F.Cu") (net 3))
 (segment (start 102.48052 52.34052) (end 101.88 51.74) (width 0.5) (layer "F.Cu") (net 15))
 (segment (start 102.48052 59.9993) (end 102.48052 52.34052) (width 0.5) (layer "F.Cu") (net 15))
 (segment (start 85.12 53.12) (end 85.12 51.74) (width 0.5) (layer "F.Cu") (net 10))
 (segment (start 89.78052 57.78052) (end 85.12 53.12) (width 0.5) (layer "F.Cu") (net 10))
 (segment (start 89.78052 59.9993) (end 89.78052 57.78052) (width 0.5) (layer "F.Cu") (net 10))
 (segment (start 67.91982 73.5) (end 79.62052 61.7993) (width 0.5) (layer "F.Cu") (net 5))
 (segment (start 55.92 80.93) (end 63.35 73.5) (width 0.5) (layer "F.Cu") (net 5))
 (segment (start 55.92 87.5) (end 55.92 80.93) (width 0.5) (layer "F.Cu") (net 5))
 (segment (start 79.62052 61.7993) (end 79.62052 59.9993) (width 0.5) (layer "F.Cu") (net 5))
 (segment (start 63.35 73.5) (end 67.91982 73.5) (width 0.5) (layer "F.Cu") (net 5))
 (segment (start 89.18 100) (end 89.18 69.55878) (width 0.5) (layer "B.Cu") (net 5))
 (segment (start 89.18 69.55878) (end 79.62052 59.9993) (width 0.5) (layer "B.Cu") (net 5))
 (segment (start 92.74 47.24) (end 92.74 51.74) (width 0.5) (layer "F.Cu") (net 1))
 (segment (start 93 51.48) (end 92.74 51.74) (width 0.5) (layer "F.Cu") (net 1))
 (segment (start 90.75 45.25) (end 92.74 47.24) (width 0.5) (layer "F.Cu") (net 1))
 (segment (start 66.1 48) (end 76.3 48) (width 0.5) (layer "F.Cu") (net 8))
 (segment (start 76.3 48) (end 80.04 51.74) (width 0.5) (layer "F.Cu") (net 8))
 (segment (start 65.1 47) (end 66.1 48) (width 0.5) (layer "F.Cu") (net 8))
 (segment (start 107.56052 52.34052) (end 106.96 51.74) (width 0.5) (layer "F.Cu") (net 17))
 (segment (start 107.56052 59.9993) (end 107.56052 52.34052) (width 0.5) (layer "F.Cu") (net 17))
 (segment (start 86 87.5) (end 112.64052 60.85948) (width 0.5) (layer "F.Cu") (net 6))
 (segment (start 66.08 87.5) (end 86 87.5) (width 0.5) (layer "F.Cu") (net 6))
 (segment (start 112.64052 60.85948) (end 112.64052 59.9993) (width 0.5) (layer "F.Cu") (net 6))
 (segment (start 62.5 83.5) (end 82.16052 63.83948) (width 0.5) (layer "F.Cu") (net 4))
 (segment (start 60.85 83.5) (end 62.5 83.5) (width 0.5) (layer "F.Cu") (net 4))
 (segment (start 82.16052 63.83948) (end 82.16052 59.9993) (width 0.5) (layer "F.Cu") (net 4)))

